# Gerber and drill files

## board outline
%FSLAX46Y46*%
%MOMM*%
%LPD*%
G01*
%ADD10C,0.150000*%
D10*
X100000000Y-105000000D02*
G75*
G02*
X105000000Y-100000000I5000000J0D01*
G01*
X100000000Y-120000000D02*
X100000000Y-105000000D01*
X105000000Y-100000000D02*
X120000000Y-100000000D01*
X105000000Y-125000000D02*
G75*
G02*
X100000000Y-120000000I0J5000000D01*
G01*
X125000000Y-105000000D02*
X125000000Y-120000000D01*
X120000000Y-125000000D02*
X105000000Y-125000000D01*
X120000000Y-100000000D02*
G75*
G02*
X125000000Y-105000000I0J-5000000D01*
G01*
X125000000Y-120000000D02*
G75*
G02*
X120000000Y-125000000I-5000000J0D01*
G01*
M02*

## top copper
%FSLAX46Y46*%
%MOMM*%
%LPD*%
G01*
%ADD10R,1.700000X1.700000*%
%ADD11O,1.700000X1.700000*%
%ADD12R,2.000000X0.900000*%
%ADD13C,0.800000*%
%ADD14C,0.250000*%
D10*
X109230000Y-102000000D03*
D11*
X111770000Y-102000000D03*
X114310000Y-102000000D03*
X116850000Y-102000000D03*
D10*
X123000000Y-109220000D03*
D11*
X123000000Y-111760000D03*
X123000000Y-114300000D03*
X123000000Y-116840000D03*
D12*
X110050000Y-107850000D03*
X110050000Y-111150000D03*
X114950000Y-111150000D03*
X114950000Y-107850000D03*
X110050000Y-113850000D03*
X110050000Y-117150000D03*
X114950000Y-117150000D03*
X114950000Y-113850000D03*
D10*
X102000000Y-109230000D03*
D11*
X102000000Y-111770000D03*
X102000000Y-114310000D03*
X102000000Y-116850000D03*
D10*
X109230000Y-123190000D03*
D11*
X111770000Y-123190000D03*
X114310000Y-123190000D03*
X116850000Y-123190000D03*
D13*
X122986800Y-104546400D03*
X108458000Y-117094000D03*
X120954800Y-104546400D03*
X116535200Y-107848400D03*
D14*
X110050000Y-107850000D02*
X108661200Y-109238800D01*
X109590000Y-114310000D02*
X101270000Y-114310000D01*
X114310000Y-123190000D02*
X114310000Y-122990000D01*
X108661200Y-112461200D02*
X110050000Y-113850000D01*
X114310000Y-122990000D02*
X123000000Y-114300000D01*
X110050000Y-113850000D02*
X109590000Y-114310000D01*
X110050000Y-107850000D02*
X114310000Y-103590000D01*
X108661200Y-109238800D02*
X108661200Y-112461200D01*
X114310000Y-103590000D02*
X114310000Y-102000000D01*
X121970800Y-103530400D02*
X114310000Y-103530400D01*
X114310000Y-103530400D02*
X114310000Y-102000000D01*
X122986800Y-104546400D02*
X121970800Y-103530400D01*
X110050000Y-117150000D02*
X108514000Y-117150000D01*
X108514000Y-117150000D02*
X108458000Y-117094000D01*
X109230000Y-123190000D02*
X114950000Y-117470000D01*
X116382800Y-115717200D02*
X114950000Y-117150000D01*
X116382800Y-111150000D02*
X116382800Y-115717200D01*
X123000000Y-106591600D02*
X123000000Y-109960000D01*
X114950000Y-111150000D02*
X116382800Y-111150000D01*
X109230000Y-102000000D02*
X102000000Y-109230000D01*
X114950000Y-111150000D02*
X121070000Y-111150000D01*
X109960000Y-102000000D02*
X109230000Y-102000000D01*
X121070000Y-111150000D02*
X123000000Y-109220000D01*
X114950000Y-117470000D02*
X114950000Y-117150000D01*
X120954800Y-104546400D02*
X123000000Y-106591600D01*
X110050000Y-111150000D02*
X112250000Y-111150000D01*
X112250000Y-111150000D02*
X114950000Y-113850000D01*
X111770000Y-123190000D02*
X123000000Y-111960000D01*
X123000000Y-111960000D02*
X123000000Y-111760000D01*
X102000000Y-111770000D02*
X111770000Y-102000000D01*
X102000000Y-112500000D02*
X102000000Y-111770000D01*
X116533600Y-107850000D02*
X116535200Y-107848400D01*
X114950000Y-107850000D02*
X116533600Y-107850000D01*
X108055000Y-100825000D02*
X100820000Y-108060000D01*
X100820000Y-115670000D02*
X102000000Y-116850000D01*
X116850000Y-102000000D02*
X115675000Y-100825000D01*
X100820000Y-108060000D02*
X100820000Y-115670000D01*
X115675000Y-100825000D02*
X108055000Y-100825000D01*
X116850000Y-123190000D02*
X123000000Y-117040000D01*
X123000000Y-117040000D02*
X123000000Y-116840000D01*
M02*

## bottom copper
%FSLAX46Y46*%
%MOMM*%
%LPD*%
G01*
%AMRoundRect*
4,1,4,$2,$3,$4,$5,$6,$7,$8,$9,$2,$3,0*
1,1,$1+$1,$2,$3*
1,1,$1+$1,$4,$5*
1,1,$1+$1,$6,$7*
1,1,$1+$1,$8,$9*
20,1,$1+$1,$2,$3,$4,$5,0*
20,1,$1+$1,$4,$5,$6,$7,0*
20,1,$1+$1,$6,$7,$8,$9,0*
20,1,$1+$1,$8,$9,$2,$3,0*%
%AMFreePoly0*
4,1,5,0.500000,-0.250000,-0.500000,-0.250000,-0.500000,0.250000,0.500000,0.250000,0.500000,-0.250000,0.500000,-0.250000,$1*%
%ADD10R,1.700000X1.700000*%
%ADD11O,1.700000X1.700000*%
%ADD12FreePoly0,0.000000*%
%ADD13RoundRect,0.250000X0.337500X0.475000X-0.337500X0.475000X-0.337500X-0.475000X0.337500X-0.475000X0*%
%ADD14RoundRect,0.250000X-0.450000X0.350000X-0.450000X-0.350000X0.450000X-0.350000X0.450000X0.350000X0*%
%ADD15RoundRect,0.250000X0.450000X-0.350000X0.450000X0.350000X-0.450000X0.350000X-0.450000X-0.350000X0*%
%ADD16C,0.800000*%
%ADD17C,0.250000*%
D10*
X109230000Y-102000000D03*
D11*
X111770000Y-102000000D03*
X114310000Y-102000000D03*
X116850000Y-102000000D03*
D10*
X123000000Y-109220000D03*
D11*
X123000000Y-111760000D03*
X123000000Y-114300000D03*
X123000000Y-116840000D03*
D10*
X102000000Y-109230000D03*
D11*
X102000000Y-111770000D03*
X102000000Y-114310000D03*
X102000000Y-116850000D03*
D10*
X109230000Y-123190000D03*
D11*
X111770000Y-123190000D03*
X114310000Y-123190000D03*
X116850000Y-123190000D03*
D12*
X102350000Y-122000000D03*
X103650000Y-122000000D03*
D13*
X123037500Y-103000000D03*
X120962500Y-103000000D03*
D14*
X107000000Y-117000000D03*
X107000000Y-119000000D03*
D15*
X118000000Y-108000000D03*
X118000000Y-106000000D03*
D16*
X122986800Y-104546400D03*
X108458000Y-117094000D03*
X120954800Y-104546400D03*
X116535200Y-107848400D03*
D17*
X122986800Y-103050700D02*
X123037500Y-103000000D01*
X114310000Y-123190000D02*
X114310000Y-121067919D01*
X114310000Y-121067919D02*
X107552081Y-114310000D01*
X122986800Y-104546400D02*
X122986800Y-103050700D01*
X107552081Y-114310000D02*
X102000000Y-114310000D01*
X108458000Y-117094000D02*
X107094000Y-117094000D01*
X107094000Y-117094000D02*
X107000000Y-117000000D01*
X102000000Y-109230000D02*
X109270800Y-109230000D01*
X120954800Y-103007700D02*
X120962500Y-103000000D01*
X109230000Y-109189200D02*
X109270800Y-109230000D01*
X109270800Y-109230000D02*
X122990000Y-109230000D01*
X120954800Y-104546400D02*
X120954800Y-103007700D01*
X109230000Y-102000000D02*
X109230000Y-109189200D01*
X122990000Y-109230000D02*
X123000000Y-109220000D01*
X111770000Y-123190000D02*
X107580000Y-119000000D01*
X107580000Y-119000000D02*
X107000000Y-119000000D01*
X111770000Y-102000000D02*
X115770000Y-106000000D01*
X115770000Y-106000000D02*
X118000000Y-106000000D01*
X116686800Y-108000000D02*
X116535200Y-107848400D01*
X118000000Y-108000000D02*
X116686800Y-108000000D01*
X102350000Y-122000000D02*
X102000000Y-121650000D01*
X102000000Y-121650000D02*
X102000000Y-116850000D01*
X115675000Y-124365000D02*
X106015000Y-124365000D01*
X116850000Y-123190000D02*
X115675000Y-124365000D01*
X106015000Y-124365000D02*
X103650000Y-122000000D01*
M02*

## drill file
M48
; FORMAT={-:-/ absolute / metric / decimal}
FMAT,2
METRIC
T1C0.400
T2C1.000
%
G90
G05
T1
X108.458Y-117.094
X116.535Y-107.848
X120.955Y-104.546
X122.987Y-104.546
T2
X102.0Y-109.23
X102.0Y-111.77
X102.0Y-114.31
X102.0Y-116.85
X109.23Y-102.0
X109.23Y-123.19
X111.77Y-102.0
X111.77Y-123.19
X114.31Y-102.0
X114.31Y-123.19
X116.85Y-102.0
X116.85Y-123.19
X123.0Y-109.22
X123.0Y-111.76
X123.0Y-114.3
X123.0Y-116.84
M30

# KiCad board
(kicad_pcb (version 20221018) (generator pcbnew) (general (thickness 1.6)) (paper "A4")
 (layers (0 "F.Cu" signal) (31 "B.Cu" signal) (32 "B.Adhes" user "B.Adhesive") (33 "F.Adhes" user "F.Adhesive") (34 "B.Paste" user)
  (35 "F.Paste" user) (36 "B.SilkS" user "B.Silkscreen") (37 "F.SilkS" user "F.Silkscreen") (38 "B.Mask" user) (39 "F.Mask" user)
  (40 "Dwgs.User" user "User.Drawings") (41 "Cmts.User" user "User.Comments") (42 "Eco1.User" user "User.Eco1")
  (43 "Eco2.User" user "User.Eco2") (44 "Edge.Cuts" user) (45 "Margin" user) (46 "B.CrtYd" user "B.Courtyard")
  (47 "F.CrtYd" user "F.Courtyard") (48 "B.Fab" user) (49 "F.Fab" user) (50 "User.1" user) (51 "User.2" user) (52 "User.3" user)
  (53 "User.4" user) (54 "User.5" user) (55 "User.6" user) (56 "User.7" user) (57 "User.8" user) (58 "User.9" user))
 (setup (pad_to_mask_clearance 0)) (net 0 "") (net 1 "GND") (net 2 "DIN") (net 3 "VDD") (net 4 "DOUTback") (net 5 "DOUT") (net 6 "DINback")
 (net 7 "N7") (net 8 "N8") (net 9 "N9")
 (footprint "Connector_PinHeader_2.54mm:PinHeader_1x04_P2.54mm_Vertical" (layer "F.Cu") (at 109.23 102 90)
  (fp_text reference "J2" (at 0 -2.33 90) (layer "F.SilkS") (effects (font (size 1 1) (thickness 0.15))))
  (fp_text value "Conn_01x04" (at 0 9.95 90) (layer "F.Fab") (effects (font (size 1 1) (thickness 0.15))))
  (pad "1" thru_hole rect (at 0 0 90) (size 1.7 1.7) (drill 1) (layers "*.Cu" "*.Mask") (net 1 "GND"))
  (pad "2" thru_hole oval (at 0 2.54 90) (size 1.7 1.7) (drill 1) (layers "*.Cu" "*.Mask") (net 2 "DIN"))
  (pad "3" thru_hole oval (at 0 5.08 90) (size 1.7 1.7) (drill 1) (layers "*.Cu" "*.Mask") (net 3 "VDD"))
  (pad "4" thru_hole oval (at 0 7.62 90) (size 1.7 1.7) (drill 1) (layers "*.Cu" "*.Mask") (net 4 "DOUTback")))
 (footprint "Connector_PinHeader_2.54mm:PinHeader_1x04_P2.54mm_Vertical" (layer "F.Cu") (at 123 109.22)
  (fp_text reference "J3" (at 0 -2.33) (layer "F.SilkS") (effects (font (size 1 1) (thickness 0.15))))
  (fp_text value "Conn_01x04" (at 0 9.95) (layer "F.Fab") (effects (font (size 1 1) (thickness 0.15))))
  (pad "1" thru_hole rect (at 0 0) (size 1.7 1.7) (drill 1) (layers "*.Cu" "*.Mask") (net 1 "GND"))
  (pad "2" thru_hole oval (at 0 2.54) (size 1.7 1.7) (drill 1) (layers "*.Cu" "*.Mask") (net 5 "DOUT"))
  (pad "3" thru_hole oval (at 0 5.08) (size 1.7 1.7) (drill 1) (layers "*.Cu" "*.Mask") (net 3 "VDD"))
  (pad "4" thru_hole oval (at 0 7.62) (size 1.7 1.7) (drill 1) (layers "*.Cu" "*.Mask") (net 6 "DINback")))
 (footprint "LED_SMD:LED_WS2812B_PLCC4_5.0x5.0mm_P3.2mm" (layer "F.Cu") (at 112.5 109.5)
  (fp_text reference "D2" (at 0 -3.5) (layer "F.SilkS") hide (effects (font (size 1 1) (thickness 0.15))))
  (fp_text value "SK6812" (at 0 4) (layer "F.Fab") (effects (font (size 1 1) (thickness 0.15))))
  (pad "1" smd rect (at -2.45 -1.65) (size 2 0.9) (layers "F.Cu" "F.Paste" "F.Mask") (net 3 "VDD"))
  (pad "2" smd rect (at -2.45 1.65) (size 2 0.9) (layers "F.Cu" "F.Paste" "F.Mask") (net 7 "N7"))
  (pad "3" smd rect (at 2.45 1.65) (size 2 0.9) (layers "F.Cu" "F.Paste" "F.Mask") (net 1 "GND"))
  (pad "4" smd rect (at 2.45 -1.65) (size 2 0.9) (layers "F.Cu" "F.Paste" "F.Mask") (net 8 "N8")))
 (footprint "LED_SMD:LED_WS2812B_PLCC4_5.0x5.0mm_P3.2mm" (layer "F.Cu") (at 112.5 115.5)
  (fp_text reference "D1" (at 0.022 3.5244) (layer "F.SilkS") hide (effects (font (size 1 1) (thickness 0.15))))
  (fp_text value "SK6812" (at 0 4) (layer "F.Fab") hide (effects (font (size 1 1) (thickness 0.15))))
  (pad "1" smd rect (at -2.45 -1.65) (size 2 0.9) (layers "F.Cu" "F.Paste" "F.Mask") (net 3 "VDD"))
  (pad "2" smd rect (at -2.45 1.65) (size 2 0.9) (layers "F.Cu" "F.Paste" "F.Mask") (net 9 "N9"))
  (pad "3" smd rect (at 2.45 1.65) (size 2 0.9) (layers "F.Cu" "F.Paste" "F.Mask") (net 1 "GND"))
  (pad "4" smd rect (at 2.45 -1.65) (size 2 0.9) (layers "F.Cu" "F.Paste" "F.Mask") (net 7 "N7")))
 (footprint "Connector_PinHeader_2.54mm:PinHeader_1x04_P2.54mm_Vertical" (layer "F.Cu") (at 102 109.23)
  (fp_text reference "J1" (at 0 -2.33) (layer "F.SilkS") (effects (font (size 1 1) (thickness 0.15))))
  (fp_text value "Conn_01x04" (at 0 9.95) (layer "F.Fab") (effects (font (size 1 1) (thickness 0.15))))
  (pad "1" thru_hole rect (at 0 0) (size 1.7 1.7) (drill 1) (layers "*.Cu" "*.Mask") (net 1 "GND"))
  (pad "2" thru_hole oval (at 0 2.54) (size 1.7 1.7) (drill 1) (layers "*.Cu" "*.Mask") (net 2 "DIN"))
  (pad "3" thru_hole oval (at 0 5.08) (size 1.7 1.7) (drill 1) (layers "*.Cu" "*.Mask") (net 3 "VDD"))
  (pad "4" thru_hole oval (at 0 7.62) (size 1.7 1.7) (drill 1) (layers "*.Cu" "*.Mask") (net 4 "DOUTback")))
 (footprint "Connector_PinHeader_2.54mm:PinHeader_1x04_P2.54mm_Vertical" (layer "F.Cu") (at 109.23 123.19 90)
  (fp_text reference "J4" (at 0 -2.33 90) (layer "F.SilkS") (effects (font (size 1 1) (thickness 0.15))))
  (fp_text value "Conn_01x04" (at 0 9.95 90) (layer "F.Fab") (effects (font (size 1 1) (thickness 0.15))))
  (pad "1" thru_hole rect (at 0 0 90) (size 1.7 1.7) (drill 1) (layers "*.Cu" "*.Mask") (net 1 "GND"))
  (pad "2" thru_hole oval (at 0 2.54 90) (size 1.7 1.7) (drill 1) (layers "*.Cu" "*.Mask") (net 5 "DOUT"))
  (pad "3" thru_hole oval (at 0 5.08 90) (size 1.7 1.7) (drill 1) (layers "*.Cu" "*.Mask") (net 3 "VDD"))
  (pad "4" thru_hole oval (at 0 7.62 90) (size 1.7 1.7) (drill 1) (layers "*.Cu" "*.Mask") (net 6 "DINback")))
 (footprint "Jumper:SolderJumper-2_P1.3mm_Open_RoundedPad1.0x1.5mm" (layer "B.Cu") (at 103 122)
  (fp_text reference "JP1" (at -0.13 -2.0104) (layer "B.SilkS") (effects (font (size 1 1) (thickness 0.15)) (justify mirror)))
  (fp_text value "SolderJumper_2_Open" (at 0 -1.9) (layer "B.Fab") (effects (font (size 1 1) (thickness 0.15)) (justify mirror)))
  (pad "1" smd custom (at -0.65 0) (size 1 0.5) (layers "B.Cu" "B.Mask") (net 4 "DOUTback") (zone_connect 2) (thermal_bridge_angle 45)
   (options (clearance outline) (anchor rect)) (primitives))
  (pad "2" smd custom (at 0.65 0) (size 1 0.5) (layers "B.Cu" "B.Mask") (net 6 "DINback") (zone_connect 2) (thermal_bridge_angle 45)
   (options (clearance outline) (anchor rect)) (primitives)))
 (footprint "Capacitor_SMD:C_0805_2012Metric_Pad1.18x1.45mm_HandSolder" (layer "B.Cu") (at 122 103 180)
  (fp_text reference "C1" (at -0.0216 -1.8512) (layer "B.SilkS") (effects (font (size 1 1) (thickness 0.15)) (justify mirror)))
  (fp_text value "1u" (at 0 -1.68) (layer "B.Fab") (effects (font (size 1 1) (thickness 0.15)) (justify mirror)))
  (pad "1" smd roundrect (at -1.0375 0 180) (size 1.175 1.45) (layers "B.Cu" "B.Paste" "B.Mask") (roundrect_rratio 0.2127659574)
   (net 3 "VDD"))
  (pad "2" smd roundrect (at 1.0375 0 180) (size 1.175 1.45) (layers "B.Cu" "B.Paste" "B.Mask") (roundrect_rratio 0.2127659574)
   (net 1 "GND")))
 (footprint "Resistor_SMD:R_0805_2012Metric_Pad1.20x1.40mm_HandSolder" (layer "B.Cu") (at 107 118 -90)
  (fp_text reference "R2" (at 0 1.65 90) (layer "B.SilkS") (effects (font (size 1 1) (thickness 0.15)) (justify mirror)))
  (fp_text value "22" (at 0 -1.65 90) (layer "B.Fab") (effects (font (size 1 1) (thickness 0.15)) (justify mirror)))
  (pad "1" smd roundrect (at -1 0 270) (size 1.2 1.4) (layers "B.Cu" "B.Paste" "B.Mask") (roundrect_rratio 0.2083333333) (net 9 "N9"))
  (pad "2" smd roundrect (at 1 0 270) (size 1.2 1.4) (layers "B.Cu" "B.Paste" "B.Mask") (roundrect_rratio 0.2083333333) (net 5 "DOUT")))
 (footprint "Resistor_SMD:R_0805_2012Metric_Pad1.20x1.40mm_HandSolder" (layer "B.Cu") (at 118 107 90)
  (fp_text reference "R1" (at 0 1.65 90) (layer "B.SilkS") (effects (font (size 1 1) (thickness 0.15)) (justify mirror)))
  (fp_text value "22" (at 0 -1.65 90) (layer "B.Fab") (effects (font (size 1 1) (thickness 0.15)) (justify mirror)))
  (pad "1" smd roundrect (at -1 0 90) (size 1.2 1.4) (layers "B.Cu" "B.Paste" "B.Mask") (roundrect_rratio 0.2083333333) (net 8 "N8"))
  (pad "2" smd roundrect (at 1 0 90) (size 1.2 1.4) (layers "B.Cu" "B.Paste" "B.Mask") (roundrect_rratio 0.2083333333) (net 2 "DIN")))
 (gr_arc (start 100 105) (mid 101.464464 101.464465) (end 105 100) (stroke (width 0.15) (type default)) (layer "Edge.Cuts"))
 (gr_line (start 100 120) (end 100 105) (stroke (width 0.15) (type default)) (layer "Edge.Cuts"))
 (gr_line (start 105 100) (end 120 100) (stroke (width 0.15) (type default)) (layer "Edge.Cuts"))
 (gr_arc (start 105 125) (mid 101.464467 123.535534) (end 100 120) (stroke (width 0.15) (type default)) (layer "Edge.Cuts"))
 (gr_line (start 125 105) (end 125 120) (stroke (width 0.15) (type default)) (layer "Edge.Cuts"))
 (gr_line (start 120 125) (end 105 125) (stroke (width 0.15) (type default)) (layer "Edge.Cuts"))
 (gr_arc (start 120 100) (mid 123.535533 101.464466) (end 125 105) (stroke (width 0.15) (type default)) (layer "Edge.Cuts"))
 (gr_arc (start 125 120) (mid 123.535534 123.535533) (end 120 125) (stroke (width 0.15) (type default)) (layer "Edge.Cuts"))
 (segment (start 110.05 107.85) (end 108.6612 109.2388) (width 0.25) (layer "F.Cu") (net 3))
 (segment (start 109.59 114.31) (end 101.27 114.31) (width 0.25) (layer "F.Cu") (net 3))
 (segment (start 114.31 123.19) (end 114.31 122.99) (width 0.25) (layer "F.Cu") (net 3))
 (segment (start 108.6612 112.4612) (end 110.05 113.85) (width 0.25) (layer "F.Cu") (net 3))
 (segment (start 114.31 122.99) (end 123 114.3) (width 0.25) (layer "F.Cu") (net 3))
 (segment (start 110.05 113.85) (end 109.59 114.31) (width 0.25) (layer "F.Cu") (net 3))
 (segment (start 110.05 107.85) (end 114.31 103.59) (width 0.25) (layer "F.Cu") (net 3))
 (segment (start 108.6612 109.2388) (end 108.6612 112.4612) (width 0.25) (layer "F.Cu") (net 3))
 (segment (start 114.31 103.59) (end 114.31 102) (width 0.25) (layer "F.Cu") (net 3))
 (segment (start 121.9708 103.5304) (end 114.31 103.5304) (width 0.25) (layer "F.Cu") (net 3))
 (segment (start 114.31 103.5304) (end 114.31 102) (width 0.25) (layer "F.Cu") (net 3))
 (segment (start 122.9868 104.5464) (end 121.9708 103.5304) (width 0.25) (layer "F.Cu") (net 3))
 (via (at 122.9868 104.5464) (size 0.8) (drill 0.4) (layers "F.Cu" "B.Cu") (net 3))
 (segment (start 122.9868 103.0507) (end 123.0375 103) (width 0.25) (layer "B.Cu") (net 3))
 (segment (start 114.31 123.19) (end 114.31 121.067919) (width 0.25) (layer "B.Cu") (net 3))
 (segment (start 114.31 121.067919) (end 107.552081 114.31) (width 0.25) (layer "B.Cu") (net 3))
 (segment (start 122.9868 104.5464) (end 122.9868 103.0507) (width 0.25) (layer "B.Cu") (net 3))
 (segment (start 107.552081 114.31) (end 102 114.31) (width 0.25) (layer "B.Cu") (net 3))
 (segment (start 110.05 117.15) (end 108.514 117.15) (width 0.25) (layer "F.Cu") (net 9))
 (segment (start 108.514 117.15) (end 108.458 117.094) (width 0.25) (layer "F.Cu") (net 9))
 (via (at 108.458 117.094) (size 0.8) (drill 0.4) (layers "F.Cu" "B.Cu") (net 9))
 (segment (start 108.458 117.094) (end 107.094 117.094) (width 0.25) (layer "B.Cu") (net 9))
 (segment (start 107.094 117.094) (end 107 117) (width 0.25) (layer "B.Cu") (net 9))
 (segment (start 109.23 123.19) (end 114.95 117.47) (width 0.25) (layer "F.Cu") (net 1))
 (segment (start 116.3828 115.7172) (end 114.95 117.15) (width 0.25) (layer "F.Cu") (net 1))
 (segment (start 116.3828 111.15) (end 116.3828 115.7172) (width 0.25) (layer "F.Cu") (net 1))
 (segment (start 123 106.5916) (end 123 109.96) (width 0.25) (layer "F.Cu") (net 1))
 (segment (start 114.95 111.15) (end 116.3828 111.15) (width 0.25) (layer "F.Cu") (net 1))
 (segment (start 109.23 102) (end 102 109.23) (width 0.25) (layer "F.Cu") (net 1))
 (segment (start 114.95 111.15) (end 121.07 111.15) (width 0.25) (layer "F.Cu") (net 1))
 (segment (start 109.96 102) (end 109.23 102) (width 0.25) (layer "F.Cu") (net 1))
 (segment (start 121.07 111.15) (end 123 109.22) (width 0.25) (layer "F.Cu") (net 1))
 (segment (start 114.95 117.47) (end 114.95 117.15) (width 0.25) (layer "F.Cu") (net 1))
 (segment (start 120.9548 104.5464) (end 123 106.5916) (width 0.25) (layer "F.Cu") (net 1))
 (via (at 120.9548 104.5464) (size 0.8) (drill 0.4) (layers "F.Cu" "B.Cu") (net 1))
 (segment (start 102 109.23) (end 109.2708 109.23) (width 0.25) (layer "B.Cu") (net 1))
 (segment (start 120.9548 103.0077) (end 120.9625 103) (width 0.25) (layer "B.Cu") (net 1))
 (segment (start 109.23 109.1892) (end 109.2708 109.23) (width 0.25) (layer "B.Cu") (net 1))
 (segment (start 109.2708 109.23) (end 122.99 109.23) (width 0.25) (layer "B.Cu") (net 1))
 (segment (start 120.9548 104.5464) (end 120.9548 103.0077) (width 0.25) (layer "B.Cu") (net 1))
 (segment (start 109.23 102) (end 109.23 109.1892) (width 0.25) (layer "B.Cu") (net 1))
 (segment (start 122.99 109.23) (end 123 109.22) (width 0.25) (layer "B.Cu") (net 1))
 (segment (start 110.05 111.15) (end 112.25 111.15) (width 0.25) (layer "F.Cu") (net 7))
 (segment (start 112.25 111.15) (end 114.95 113.85) (width 0.25) (layer "F.Cu") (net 7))
 (segment (start 111.77 123.19) (end 123 111.96) (width 0.25) (layer "F.Cu") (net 5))
 (segment (start 123 111.96) (end 123 111.76) (width 0.25) (layer "F.Cu") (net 5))
 (segment (start 111.77 123.19) (end 107.58 119) (width 0.25) (layer "B.Cu") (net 5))
 (segment (start 107.58 119) (end 107 119) (width 0.25) (layer "B.Cu") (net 5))
 (segment (start 102 111.77) (end 111.77 102) (width 0.25) (layer "F.Cu") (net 2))
 (segment (start 102 112.5) (end 102 111.77) (width 0.25) (layer "F.Cu") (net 2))
 (segment (start 111.77 102) (end 115.77 106) (width 0.25) (layer "B.Cu") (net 2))
 (segment (start 115.77 106) (end 118 106) (width 0.25) (layer "B.Cu") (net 2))
 (segment (start 116.5336 107.85) (end 116.5352 107.8484) (width 0.25) (layer "F.Cu") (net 8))
 (segment (start 114.95 107.85) (end 116.5336 107.85) (width 0.25) (layer "F.Cu") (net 8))
 (via (at 116.5352 107.8484) (size 0.8) (drill 0.4) (layers "F.Cu" "B.Cu") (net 8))
 (segment (start 116.6868 108) (end 116.5352 107.8484) (width 0.25) (layer "B.Cu") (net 8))
 (segment (start 118 108) (end 116.6868 108) (width 0.25) (layer "B.Cu") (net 8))
 (segment (start 108.055 100.825) (end 100.82 108.06) (width 0.25) (layer "F.Cu") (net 4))
 (segment (start 100.82 115.67) (end 102 116.85) (width 0.25) (layer "F.Cu") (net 4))
 (segment (start 116.85 102) (end 115.675 100.825) (width 0.25) (layer "F.Cu") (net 4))
 (segment (start 100.82 108.06) (end 100.82 115.67) (width 0.25) (layer "F.Cu") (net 4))
 (segment (start 115.675 100.825) (end 108.055 100.825) (width 0.25) (layer "F.Cu") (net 4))
 (segment (start 102.35 122) (end 102 121.65) (width 0.25) (layer "B.Cu") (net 4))
 (segment (start 102 121.65) (end 102 116.85) (width 0.25) (layer "B.Cu") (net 4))
 (segment (start 116.85 123.19) (end 123 117.04) (width 0.25) (layer "F.Cu") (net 6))
 (segment (start 123 117.04) (end 123 116.84) (width 0.25) (layer "F.Cu") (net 6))
 (segment (start 115.675 124.365) (end 106.015 124.365) (width 0.25) (layer "B.Cu") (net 6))
 (segment (start 116.85 123.19) (end 115.675 124.365) (width 0.25) (layer "B.Cu") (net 6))
 (segment (start 106.015 124.365) (end 103.65 122) (width 0.25) (layer "B.Cu") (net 6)))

